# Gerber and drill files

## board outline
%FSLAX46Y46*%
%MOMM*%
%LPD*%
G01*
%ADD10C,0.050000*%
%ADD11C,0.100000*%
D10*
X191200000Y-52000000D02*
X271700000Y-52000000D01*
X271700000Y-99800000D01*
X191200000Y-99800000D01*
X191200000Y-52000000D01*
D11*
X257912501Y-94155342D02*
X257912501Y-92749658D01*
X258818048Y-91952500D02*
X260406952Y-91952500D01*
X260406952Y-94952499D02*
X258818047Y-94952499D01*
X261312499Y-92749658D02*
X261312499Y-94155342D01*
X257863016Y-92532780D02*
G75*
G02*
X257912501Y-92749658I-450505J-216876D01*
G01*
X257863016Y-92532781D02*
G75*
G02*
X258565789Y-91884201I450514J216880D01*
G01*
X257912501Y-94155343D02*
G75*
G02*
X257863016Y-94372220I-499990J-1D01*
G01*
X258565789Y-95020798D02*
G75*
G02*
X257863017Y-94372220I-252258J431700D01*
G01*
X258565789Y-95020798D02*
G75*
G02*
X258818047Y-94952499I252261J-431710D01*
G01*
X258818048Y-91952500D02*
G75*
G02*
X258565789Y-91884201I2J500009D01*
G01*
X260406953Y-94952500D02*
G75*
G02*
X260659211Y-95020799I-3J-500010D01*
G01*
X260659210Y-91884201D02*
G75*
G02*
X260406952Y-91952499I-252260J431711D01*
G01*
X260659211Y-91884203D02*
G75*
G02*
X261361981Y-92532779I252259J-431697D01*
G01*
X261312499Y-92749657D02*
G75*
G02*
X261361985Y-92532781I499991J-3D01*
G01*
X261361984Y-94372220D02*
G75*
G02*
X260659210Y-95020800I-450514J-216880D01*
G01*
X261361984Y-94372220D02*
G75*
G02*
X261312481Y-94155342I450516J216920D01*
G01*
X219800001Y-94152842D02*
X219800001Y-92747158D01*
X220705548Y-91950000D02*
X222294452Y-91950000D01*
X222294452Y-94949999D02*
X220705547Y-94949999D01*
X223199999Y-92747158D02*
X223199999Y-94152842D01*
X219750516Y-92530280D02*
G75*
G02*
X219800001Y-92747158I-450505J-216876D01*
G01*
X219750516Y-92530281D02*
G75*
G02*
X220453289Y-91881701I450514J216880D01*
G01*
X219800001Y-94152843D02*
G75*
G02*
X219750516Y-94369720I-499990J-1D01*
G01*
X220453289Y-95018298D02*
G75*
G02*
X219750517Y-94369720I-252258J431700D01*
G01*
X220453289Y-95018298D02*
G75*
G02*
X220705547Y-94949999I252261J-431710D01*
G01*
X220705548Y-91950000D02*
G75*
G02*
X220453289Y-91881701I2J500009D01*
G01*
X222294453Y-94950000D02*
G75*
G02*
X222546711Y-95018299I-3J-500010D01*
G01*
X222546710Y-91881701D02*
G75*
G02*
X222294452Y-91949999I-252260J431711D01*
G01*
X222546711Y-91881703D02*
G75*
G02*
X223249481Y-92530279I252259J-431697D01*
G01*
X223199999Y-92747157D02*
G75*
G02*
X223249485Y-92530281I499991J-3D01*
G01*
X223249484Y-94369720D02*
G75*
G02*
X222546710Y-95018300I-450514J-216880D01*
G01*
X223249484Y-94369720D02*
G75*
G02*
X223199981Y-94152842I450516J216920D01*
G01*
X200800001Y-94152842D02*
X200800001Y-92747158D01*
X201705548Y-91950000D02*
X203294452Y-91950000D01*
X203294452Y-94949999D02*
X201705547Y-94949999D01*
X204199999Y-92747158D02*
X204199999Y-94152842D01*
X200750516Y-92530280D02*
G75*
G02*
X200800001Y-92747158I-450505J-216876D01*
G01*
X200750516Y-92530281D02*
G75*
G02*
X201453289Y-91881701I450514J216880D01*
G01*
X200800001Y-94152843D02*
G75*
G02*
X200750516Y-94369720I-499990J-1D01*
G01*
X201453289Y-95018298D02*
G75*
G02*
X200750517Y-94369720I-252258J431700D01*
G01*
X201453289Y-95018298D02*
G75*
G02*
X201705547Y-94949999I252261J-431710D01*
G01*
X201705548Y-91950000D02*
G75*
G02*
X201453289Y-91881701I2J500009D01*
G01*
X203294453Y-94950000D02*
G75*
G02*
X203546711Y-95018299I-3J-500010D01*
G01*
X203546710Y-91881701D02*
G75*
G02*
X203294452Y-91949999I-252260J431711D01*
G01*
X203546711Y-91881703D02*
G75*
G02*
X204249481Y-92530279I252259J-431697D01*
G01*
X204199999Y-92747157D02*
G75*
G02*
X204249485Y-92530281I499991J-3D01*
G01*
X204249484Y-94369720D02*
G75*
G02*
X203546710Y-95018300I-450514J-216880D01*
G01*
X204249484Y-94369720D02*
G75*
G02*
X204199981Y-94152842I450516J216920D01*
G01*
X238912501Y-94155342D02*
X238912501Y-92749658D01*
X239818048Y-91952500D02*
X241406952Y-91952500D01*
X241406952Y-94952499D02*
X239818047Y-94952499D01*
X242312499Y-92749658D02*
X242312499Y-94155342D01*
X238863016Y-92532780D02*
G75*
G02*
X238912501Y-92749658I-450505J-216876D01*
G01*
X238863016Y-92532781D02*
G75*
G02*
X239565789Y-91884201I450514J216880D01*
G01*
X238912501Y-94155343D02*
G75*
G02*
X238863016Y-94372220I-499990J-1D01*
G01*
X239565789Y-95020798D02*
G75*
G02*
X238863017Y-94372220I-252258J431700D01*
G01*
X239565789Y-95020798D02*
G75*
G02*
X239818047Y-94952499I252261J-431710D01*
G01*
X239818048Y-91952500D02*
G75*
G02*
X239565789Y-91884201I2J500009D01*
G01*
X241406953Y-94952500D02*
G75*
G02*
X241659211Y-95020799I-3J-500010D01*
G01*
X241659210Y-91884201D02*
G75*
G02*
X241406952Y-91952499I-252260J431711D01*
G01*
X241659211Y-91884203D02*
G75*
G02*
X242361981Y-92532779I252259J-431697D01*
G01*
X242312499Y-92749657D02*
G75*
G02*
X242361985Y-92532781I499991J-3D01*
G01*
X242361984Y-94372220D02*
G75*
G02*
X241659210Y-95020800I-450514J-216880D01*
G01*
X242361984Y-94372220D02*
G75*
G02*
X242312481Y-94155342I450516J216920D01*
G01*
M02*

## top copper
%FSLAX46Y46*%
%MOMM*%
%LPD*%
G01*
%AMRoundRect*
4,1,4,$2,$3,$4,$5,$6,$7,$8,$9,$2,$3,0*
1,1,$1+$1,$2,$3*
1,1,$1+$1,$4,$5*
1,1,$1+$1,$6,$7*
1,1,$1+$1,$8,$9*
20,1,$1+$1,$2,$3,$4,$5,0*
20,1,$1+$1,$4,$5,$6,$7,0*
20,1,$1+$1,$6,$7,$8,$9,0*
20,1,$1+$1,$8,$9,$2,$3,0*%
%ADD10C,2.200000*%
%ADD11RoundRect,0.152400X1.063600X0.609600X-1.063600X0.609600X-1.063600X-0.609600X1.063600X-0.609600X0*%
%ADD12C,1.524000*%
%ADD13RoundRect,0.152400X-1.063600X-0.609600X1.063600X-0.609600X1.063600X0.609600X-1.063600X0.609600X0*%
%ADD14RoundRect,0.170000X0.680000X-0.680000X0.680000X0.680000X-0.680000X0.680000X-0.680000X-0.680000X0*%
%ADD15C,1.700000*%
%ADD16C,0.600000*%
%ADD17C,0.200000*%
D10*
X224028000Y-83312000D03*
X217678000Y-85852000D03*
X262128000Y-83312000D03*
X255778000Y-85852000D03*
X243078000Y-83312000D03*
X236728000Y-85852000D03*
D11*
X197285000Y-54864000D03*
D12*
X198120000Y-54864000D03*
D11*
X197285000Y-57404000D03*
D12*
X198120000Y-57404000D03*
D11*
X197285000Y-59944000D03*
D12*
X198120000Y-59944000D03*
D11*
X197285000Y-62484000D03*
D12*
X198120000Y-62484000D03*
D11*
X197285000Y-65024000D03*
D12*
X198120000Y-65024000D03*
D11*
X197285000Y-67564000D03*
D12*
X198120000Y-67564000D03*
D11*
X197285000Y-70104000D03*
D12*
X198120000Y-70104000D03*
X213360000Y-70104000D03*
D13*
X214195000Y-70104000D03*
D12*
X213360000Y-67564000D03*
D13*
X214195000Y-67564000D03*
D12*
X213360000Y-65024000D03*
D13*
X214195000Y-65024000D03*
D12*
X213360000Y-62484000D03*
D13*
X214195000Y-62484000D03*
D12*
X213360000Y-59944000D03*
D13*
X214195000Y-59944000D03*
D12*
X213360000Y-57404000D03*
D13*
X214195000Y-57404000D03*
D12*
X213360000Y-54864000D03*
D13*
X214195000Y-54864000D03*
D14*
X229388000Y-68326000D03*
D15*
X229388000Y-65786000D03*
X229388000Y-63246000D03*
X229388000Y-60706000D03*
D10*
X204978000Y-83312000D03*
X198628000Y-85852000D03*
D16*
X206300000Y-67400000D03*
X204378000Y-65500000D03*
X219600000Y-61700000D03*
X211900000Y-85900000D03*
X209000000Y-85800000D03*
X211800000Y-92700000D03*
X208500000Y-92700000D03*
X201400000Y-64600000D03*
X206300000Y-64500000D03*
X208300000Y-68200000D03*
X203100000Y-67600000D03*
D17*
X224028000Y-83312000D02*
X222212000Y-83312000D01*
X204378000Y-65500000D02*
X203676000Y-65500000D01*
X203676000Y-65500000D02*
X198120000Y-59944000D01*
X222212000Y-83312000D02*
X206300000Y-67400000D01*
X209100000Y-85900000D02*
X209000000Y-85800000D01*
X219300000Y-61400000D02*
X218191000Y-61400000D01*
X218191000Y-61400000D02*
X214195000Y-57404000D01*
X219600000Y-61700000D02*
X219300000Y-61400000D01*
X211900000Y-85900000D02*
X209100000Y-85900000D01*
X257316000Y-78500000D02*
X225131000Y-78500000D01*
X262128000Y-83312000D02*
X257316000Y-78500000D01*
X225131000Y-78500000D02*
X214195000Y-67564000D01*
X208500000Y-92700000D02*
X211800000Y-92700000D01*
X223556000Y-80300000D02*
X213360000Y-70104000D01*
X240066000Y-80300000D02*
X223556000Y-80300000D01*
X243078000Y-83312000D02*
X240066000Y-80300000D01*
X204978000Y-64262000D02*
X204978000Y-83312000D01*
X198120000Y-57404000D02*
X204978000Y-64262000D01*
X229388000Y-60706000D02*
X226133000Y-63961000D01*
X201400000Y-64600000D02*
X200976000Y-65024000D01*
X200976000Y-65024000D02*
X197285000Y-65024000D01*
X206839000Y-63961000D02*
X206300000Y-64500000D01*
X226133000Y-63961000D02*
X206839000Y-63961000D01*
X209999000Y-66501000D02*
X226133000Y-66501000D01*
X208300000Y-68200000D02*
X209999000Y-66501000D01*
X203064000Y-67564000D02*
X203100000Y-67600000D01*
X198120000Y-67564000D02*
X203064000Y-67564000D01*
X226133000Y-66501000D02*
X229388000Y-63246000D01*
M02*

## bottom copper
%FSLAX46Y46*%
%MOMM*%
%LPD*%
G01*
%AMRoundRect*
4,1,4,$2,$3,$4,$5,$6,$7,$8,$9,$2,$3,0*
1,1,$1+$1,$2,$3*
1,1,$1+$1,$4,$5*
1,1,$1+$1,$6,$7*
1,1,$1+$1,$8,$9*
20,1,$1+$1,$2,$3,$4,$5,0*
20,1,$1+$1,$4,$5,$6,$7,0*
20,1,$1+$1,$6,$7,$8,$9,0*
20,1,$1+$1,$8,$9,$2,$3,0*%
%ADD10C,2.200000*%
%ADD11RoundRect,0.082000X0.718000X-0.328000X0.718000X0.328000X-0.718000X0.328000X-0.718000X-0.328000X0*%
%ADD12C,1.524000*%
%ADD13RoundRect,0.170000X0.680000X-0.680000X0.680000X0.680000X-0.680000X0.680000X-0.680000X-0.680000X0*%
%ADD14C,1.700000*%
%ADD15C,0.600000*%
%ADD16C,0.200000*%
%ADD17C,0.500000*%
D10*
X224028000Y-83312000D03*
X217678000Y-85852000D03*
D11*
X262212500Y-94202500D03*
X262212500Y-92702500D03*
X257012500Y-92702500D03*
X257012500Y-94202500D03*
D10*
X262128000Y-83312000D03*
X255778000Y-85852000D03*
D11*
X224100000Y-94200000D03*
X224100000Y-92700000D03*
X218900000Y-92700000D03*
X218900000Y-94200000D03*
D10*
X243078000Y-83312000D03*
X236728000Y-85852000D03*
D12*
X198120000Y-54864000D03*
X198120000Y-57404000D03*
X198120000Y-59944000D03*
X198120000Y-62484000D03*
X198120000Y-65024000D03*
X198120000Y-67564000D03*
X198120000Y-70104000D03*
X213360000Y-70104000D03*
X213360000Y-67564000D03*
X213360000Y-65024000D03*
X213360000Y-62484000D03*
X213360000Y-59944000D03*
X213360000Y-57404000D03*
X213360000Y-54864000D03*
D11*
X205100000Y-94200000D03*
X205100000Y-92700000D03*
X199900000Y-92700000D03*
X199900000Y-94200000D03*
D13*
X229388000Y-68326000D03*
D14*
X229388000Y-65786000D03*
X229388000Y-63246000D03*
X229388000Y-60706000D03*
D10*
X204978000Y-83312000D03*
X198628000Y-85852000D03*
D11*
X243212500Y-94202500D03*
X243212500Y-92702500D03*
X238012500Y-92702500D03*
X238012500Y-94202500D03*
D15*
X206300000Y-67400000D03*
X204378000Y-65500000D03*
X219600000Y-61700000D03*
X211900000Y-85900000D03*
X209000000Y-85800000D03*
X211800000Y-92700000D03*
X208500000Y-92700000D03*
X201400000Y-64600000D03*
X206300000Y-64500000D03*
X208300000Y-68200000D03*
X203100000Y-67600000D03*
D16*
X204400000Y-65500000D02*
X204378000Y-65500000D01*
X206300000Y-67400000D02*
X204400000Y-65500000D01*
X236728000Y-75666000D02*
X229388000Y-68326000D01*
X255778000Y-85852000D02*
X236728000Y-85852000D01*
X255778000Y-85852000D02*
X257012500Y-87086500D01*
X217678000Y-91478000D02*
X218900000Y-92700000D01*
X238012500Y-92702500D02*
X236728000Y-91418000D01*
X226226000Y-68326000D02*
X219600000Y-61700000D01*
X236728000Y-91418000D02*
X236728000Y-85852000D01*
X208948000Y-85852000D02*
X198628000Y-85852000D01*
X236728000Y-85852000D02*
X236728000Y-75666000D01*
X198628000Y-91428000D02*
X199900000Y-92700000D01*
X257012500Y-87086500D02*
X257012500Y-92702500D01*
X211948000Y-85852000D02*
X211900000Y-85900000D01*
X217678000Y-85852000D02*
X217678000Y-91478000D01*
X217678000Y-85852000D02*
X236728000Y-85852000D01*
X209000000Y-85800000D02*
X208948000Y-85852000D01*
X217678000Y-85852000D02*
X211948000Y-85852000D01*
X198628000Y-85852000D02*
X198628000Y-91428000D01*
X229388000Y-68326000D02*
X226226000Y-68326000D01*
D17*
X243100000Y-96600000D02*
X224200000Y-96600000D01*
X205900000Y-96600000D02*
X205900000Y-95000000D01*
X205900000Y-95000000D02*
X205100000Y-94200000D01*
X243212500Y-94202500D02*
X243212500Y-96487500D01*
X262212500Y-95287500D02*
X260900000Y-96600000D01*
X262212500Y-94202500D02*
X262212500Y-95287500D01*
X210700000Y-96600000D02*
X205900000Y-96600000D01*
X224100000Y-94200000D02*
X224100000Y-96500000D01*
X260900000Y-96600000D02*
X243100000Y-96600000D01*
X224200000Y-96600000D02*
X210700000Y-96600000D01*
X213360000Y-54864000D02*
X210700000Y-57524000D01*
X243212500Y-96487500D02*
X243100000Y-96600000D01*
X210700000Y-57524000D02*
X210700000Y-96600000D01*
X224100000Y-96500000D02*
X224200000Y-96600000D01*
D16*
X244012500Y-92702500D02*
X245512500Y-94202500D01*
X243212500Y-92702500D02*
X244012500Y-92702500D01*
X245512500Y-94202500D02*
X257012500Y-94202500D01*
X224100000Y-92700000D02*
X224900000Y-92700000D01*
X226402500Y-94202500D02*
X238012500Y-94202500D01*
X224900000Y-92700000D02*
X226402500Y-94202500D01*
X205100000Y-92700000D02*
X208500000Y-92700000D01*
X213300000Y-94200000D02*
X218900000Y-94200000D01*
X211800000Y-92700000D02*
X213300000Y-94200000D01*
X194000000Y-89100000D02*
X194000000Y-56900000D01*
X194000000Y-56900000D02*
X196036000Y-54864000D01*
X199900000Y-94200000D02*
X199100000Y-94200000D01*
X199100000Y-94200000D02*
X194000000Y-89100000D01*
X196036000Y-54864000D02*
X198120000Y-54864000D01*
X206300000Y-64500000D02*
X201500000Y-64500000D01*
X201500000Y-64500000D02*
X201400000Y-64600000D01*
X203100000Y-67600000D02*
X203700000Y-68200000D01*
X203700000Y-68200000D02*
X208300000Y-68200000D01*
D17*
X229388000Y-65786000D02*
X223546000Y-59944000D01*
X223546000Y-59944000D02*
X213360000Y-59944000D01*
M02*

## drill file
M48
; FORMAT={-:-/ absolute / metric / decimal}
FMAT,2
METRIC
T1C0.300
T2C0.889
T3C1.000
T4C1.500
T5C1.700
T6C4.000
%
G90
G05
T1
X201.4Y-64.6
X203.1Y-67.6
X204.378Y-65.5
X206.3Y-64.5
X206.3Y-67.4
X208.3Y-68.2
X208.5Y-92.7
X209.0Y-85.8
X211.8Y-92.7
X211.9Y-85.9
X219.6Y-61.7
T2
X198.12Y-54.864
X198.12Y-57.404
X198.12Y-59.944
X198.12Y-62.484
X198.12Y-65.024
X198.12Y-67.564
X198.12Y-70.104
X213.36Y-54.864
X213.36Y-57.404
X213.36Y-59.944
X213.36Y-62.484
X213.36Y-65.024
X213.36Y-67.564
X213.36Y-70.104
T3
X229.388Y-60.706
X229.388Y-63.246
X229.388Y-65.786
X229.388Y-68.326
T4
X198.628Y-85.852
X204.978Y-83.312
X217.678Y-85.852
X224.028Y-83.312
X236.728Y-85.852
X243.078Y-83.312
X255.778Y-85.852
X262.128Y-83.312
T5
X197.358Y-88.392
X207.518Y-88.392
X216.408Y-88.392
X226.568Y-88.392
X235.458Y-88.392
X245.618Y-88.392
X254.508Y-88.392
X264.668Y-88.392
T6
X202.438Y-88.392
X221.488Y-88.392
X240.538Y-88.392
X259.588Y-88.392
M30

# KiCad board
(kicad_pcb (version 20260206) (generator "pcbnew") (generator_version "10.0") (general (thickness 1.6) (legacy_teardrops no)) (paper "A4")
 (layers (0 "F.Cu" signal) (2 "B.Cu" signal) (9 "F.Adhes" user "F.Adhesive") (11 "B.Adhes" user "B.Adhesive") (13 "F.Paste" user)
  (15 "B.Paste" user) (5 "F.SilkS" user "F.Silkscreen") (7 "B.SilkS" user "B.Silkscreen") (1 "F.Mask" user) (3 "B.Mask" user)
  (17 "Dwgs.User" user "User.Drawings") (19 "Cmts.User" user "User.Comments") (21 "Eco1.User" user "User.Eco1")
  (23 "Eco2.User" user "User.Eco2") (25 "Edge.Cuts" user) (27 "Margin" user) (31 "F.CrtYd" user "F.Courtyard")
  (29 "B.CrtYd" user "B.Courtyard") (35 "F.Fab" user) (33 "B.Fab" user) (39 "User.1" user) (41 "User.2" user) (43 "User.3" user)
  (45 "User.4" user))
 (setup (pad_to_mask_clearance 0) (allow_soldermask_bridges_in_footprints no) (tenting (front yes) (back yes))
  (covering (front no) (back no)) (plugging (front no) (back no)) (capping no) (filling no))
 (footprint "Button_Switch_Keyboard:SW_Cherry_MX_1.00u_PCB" (layer "F.Cu") (at 224.028 83.312)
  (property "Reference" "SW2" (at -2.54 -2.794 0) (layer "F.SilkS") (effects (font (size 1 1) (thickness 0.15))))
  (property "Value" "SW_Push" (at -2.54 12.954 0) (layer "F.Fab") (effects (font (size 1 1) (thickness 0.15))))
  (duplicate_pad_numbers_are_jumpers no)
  (pad "" np_thru_hole circle (at -7.62 5.08) (size 1.7 1.7) (drill 1.7) (layers "*.Cu" "*.Mask"))
  (pad "" np_thru_hole circle (at -2.54 5.08) (size 4 4) (drill 4) (layers "*.Cu" "*.Mask"))
  (pad "" np_thru_hole circle (at 2.54 5.08) (size 1.7 1.7) (drill 1.7) (layers "*.Cu" "*.Mask"))
  (pad "1" thru_hole circle (at 0 0) (size 2.2 2.2) (drill 1.5) (layers "*.Cu" "*.Mask") (remove_unused_layers no)
   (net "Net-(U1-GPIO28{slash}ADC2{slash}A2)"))
  (pad "2" thru_hole circle (at -6.35 2.54) (size 2.2 2.2) (drill 1.5) (layers "*.Cu" "*.Mask") (remove_unused_layers no) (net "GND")))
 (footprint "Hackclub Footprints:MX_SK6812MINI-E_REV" (layer "F.Cu") (at 259.6125 88.3725)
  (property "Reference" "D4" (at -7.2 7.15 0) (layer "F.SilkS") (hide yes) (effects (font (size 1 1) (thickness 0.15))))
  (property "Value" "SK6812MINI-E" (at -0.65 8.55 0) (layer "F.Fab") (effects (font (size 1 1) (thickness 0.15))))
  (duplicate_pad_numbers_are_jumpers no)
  (fp_line (start -1.699999 5.782842) (end -1.699999 4.377158) (stroke (width 0.1) (type solid)) (layer "Edge.Cuts"))
  (fp_line (start -0.794452 3.58) (end 0.794452 3.58) (stroke (width 0.1) (type solid)) (layer "Edge.Cuts"))
  (fp_line (start 0.794452 6.579999) (end -0.794453 6.579999) (stroke (width 0.1) (type solid)) (layer "Edge.Cuts"))
  (fp_line (start 1.699999 4.377158) (end 1.699999 5.782842) (stroke (width 0.1) (type solid)) (layer "Edge.Cuts"))
  (fp_arc (start -1.749484 4.16028) (mid -1.712527 4.265932) (end -1.699999 4.377158) (stroke (width 0.1) (type solid)) (layer "Edge.Cuts"))
  (fp_arc (start -1.749484 4.160281) (mid -1.638072 3.575965) (end -1.046711 3.511701) (stroke (width 0.1) (type solid)) (layer "Edge.Cuts"))
  (fp_arc (start -1.699999 5.782843) (mid -1.712527 5.894068) (end -1.749484 5.99972) (stroke (width 0.1) (type solid)) (layer "Edge.Cuts"))
  (fp_arc (start -1.046711 6.648298) (mid -1.638071 6.584034) (end -1.749484 5.99972) (stroke (width 0.1) (type solid)) (layer "Edge.Cuts"))
  (fp_arc (start -1.046711 6.648298) (mid -0.925123 6.597376) (end -0.794453 6.579999) (stroke (width 0.1) (type solid)) (layer "Edge.Cuts"))
  (fp_arc (start -0.794452 3.58) (mid -0.925123 3.562623) (end -1.046711 3.511701) (stroke (width 0.1) (type solid)) (layer "Edge.Cuts"))
  (fp_arc (start 0.794453 6.58) (mid 0.925123 6.597377) (end 1.046711 6.648299) (stroke (width 0.1) (type solid)) (layer "Edge.Cuts"))
  (fp_arc (start 1.04671 3.511701) (mid 0.925122 3.562623) (end 0.794452 3.58) (stroke (width 0.1) (type solid)) (layer "Edge.Cuts"))
  (fp_arc (start 1.046711 3.511703) (mid 1.63807 3.575966) (end 1.749484 4.16028) (stroke (width 0.1) (type solid)) (layer "Edge.Cuts"))
  (fp_arc (start 1.699999 4.377157) (mid 1.712527 4.265932) (end 1.749484 4.16028) (stroke (width 0.1) (type solid)) (layer "Edge.Cuts"))
  (fp_arc (start 1.749484 5.99972) (mid 1.638071 6.584035) (end 1.046711 6.648299) (stroke (width 0.1) (type solid)) (layer "Edge.Cuts"))
  (fp_arc (start 1.749484 5.99972) (mid 1.712527 5.894068) (end 1.699999 5.782842) (stroke (width 0.1) (type solid)) (layer "Edge.Cuts"))
  (pad "1" smd roundrect (at 2.6 5.83 90) (size 0.82 1.6) (layers "B.Cu" "B.Mask" "B.Paste") (roundrect_rratio 0.1) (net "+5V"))
  (pad "2" smd roundrect (at 2.6 4.33 90) (size 0.82 1.6) (layers "B.Cu" "B.Mask" "B.Paste") (roundrect_rratio 0.1)
   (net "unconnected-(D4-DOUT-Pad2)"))
  (pad "3" smd roundrect (at -2.6 4.33 90) (size 0.82 1.6) (layers "B.Cu" "B.Mask" "B.Paste") (roundrect_rratio 0.1) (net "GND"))
  (pad "4" smd roundrect (at -2.6 5.83 90) (size 0.82 1.6) (layers "B.Cu" "B.Mask" "B.Paste") (roundrect_rratio 0.1) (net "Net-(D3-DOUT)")))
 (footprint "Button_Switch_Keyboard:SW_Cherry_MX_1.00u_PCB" (layer "F.Cu") (at 262.128 83.312)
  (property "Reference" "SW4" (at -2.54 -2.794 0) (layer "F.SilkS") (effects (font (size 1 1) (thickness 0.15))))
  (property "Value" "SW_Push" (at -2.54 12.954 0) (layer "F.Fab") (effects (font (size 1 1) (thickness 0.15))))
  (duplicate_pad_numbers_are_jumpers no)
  (pad "" np_thru_hole circle (at -7.62 5.08) (size 1.7 1.7) (drill 1.7) (layers "*.Cu" "*.Mask"))
  (pad "" np_thru_hole circle (at -2.54 5.08) (size 4 4) (drill 4) (layers "*.Cu" "*.Mask"))
  (pad "" np_thru_hole circle (at 2.54 5.08) (size 1.7 1.7) (drill 1.7) (layers "*.Cu" "*.Mask"))
  (pad "1" thru_hole circle (at 0 0) (size 2.2 2.2) (drill 1.5) (layers "*.Cu" "*.Mask") (remove_unused_layers no)
   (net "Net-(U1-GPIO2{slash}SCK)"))
  (pad "2" thru_hole circle (at -6.35 2.54) (size 2.2 2.2) (drill 1.5) (layers "*.Cu" "*.Mask") (remove_unused_layers no) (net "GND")))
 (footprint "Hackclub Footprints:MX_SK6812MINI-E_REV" (layer "F.Cu") (at 221.5 88.37)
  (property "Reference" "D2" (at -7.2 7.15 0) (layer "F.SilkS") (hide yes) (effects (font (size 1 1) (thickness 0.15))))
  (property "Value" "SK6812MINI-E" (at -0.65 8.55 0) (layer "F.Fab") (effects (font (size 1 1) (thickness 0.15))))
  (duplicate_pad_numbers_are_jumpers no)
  (fp_line (start -1.699999 5.782842) (end -1.699999 4.377158) (stroke (width 0.1) (type solid)) (layer "Edge.Cuts"))
  (fp_line (start -0.794452 3.58) (end 0.794452 3.58) (stroke (width 0.1) (type solid)) (layer "Edge.Cuts"))
  (fp_line (start 0.794452 6.579999) (end -0.794453 6.579999) (stroke (width 0.1) (type solid)) (layer "Edge.Cuts"))
  (fp_line (start 1.699999 4.377158) (end 1.699999 5.782842) (stroke (width 0.1) (type solid)) (layer "Edge.Cuts"))
  (fp_arc (start -1.749484 4.16028) (mid -1.712527 4.265932) (end -1.699999 4.377158) (stroke (width 0.1) (type solid)) (layer "Edge.Cuts"))
  (fp_arc (start -1.749484 4.160281) (mid -1.638072 3.575965) (end -1.046711 3.511701) (stroke (width 0.1) (type solid)) (layer "Edge.Cuts"))
  (fp_arc (start -1.699999 5.782843) (mid -1.712527 5.894068) (end -1.749484 5.99972) (stroke (width 0.1) (type solid)) (layer "Edge.Cuts"))
  (fp_arc (start -1.046711 6.648298) (mid -1.638071 6.584034) (end -1.749484 5.99972) (stroke (width 0.1) (type solid)) (layer "Edge.Cuts"))
  (fp_arc (start -1.046711 6.648298) (mid -0.925123 6.597376) (end -0.794453 6.579999) (stroke (width 0.1) (type solid)) (layer "Edge.Cuts"))
  (fp_arc (start -0.794452 3.58) (mid -0.925123 3.562623) (end -1.046711 3.511701) (stroke (width 0.1) (type solid)) (layer "Edge.Cuts"))
  (fp_arc (start 0.794453 6.58) (mid 0.925123 6.597377) (end 1.046711 6.648299) (stroke (width 0.1) (type solid)) (layer "Edge.Cuts"))
  (fp_arc (start 1.04671 3.511701) (mid 0.925122 3.562623) (end 0.794452 3.58) (stroke (width 0.1) (type solid)) (layer "Edge.Cuts"))
  (fp_arc (start 1.046711 3.511703) (mid 1.63807 3.575966) (end 1.749484 4.16028) (stroke (width 0.1) (type solid)) (layer "Edge.Cuts"))
  (fp_arc (start 1.699999 4.377157) (mid 1.712527 4.265932) (end 1.749484 4.16028) (stroke (width 0.1) (type solid)) (layer "Edge.Cuts"))
  (fp_arc (start 1.749484 5.99972) (mid 1.638071 6.584035) (end 1.046711 6.648299) (stroke (width 0.1) (type solid)) (layer "Edge.Cuts"))
  (fp_arc (start 1.749484 5.99972) (mid 1.712527 5.894068) (end 1.699999 5.782842) (stroke (width 0.1) (type solid)) (layer "Edge.Cuts"))
  (pad "1" smd roundrect (at 2.6 5.83 90) (size 0.82 1.6) (layers "B.Cu" "B.Mask" "B.Paste") (roundrect_rratio 0.1) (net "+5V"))
  (pad "2" smd roundrect (at 2.6 4.33 90) (size 0.82 1.6) (layers "B.Cu" "B.Mask" "B.Paste") (roundrect_rratio 0.1) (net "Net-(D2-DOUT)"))
  (pad "3" smd roundrect (at -2.6 4.33 90) (size 0.82 1.6) (layers "B.Cu" "B.Mask" "B.Paste") (roundrect_rratio 0.1) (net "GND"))
  (pad "4" smd roundrect (at -2.6 5.83 90) (size 0.82 1.6) (layers "B.Cu" "B.Mask" "B.Paste") (roundrect_rratio 0.1) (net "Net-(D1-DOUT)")))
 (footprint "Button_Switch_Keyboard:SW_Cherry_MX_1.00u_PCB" (layer "F.Cu") (at 243.078 83.312)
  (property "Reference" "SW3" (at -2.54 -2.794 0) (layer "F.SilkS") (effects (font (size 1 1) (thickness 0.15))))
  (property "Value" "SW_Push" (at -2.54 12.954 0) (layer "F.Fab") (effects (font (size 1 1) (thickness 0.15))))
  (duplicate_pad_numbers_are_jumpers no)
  (pad "" np_thru_hole circle (at -7.62 5.08) (size 1.7 1.7) (drill 1.7) (layers "*.Cu" "*.Mask"))
  (pad "" np_thru_hole circle (at -2.54 5.08) (size 4 4) (drill 4) (layers "*.Cu" "*.Mask"))
  (pad "" np_thru_hole circle (at 2.54 5.08) (size 1.7 1.7) (drill 1.7) (layers "*.Cu" "*.Mask"))
  (pad "1" thru_hole circle (at 0 0) (size 2.2 2.2) (drill 1.5) (layers "*.Cu" "*.Mask") (remove_unused_layers no)
   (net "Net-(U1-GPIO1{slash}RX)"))
  (pad "2" thru_hole circle (at -6.35 2.54) (size 2.2 2.2) (drill 1.5) (layers "*.Cu" "*.Mask") (remove_unused_layers no) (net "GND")))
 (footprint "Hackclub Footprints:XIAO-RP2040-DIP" (layer "F.Cu") (at 205.74 62.484)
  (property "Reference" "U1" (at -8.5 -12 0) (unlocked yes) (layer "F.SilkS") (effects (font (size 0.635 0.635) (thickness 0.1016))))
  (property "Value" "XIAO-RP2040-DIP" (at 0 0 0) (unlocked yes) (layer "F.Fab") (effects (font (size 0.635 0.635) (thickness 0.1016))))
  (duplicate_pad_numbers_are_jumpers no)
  (pad "1" smd roundrect (at -8.455 -7.62 180) (size 2.432 1.524) (layers "F.Cu" "F.Mask") (roundrect_rratio 0.1) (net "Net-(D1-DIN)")
   (thermal_bridge_angle 45))
  (pad "1" thru_hole circle (at -7.62 -7.62 180) (size 1.524 1.524) (drill 0.889) (layers "*.Cu" "*.Mask") (remove_unused_layers no)
   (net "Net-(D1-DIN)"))
  (pad "2" smd roundrect (at -8.455 -5.08 180) (size 2.432 1.524) (layers "F.Cu" "F.Mask") (roundrect_rratio 0.1)
   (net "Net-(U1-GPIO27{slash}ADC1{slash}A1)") (thermal_bridge_angle 45))
  (pad "2" thru_hole circle (at -7.62 -5.08 180) (size 1.524 1.524) (drill 0.889) (layers "*.Cu" "*.Mask") (remove_unused_layers no)
   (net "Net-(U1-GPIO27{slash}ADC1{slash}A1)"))
  (pad "3" smd roundrect (at -8.455 -2.54 180) (size 2.432 1.524) (layers "F.Cu" "F.Mask") (roundrect_rratio 0.1)
   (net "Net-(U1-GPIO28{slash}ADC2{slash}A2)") (thermal_bridge_angle 45))
  (pad "3" thru_hole circle (at -7.62 -2.54 180) (size 1.524 1.524) (drill 0.889) (layers "*.Cu" "*.Mask") (remove_unused_layers no)
   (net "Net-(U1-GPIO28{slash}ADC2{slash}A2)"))
  (pad "4" smd roundrect (at -8.455 0 180) (size 2.432 1.524) (layers "F.Cu" "F.Mask") (roundrect_rratio 0.1)
   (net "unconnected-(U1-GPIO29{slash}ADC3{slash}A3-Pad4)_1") (thermal_bridge_angle 45))
  (pad "4" thru_hole circle (at -7.62 0 180) (size 1.524 1.524) (drill 0.889) (layers "*.Cu" "*.Mask") (remove_unused_layers no)
   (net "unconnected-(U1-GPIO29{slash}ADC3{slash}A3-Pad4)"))
  (pad "5" smd roundrect (at -8.455 2.54 180) (size 2.432 1.524) (layers "F.Cu" "F.Mask") (roundrect_rratio 0.1) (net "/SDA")
   (thermal_bridge_angle 45))
  (pad "5" thru_hole circle (at -7.62 2.54 180) (size 1.524 1.524) (drill 0.889) (layers "*.Cu" "*.Mask") (remove_unused_layers no)
   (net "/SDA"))
  (pad "6" smd roundrect (at -8.455 5.08 180) (size 2.432 1.524) (layers "F.Cu" "F.Mask") (roundrect_rratio 0.1) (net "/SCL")
   (thermal_bridge_angle 45))
  (pad "6" thru_hole circle (at -7.62 5.08 180) (size 1.524 1.524) (drill 0.889) (layers "*.Cu" "*.Mask") (remove_unused_layers no)
   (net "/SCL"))
  (pad "7" smd roundrect (at -8.455 7.62 180) (size 2.432 1.524) (layers "F.Cu" "F.Mask") (roundrect_rratio 0.1)
   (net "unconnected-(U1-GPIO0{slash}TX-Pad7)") (thermal_bridge_angle 45))
  (pad "7" thru_hole circle (at -7.62 7.62 180) (size 1.524 1.524) (drill 0.889) (layers "*.Cu" "*.Mask") (remove_unused_layers no)
   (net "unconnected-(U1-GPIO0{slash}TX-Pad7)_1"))
  (pad "8" thru_hole circle (at 7.62 7.62) (size 1.524 1.524) (drill 0.889) (layers "*.Cu" "*.Mask") (remove_unused_layers no)
   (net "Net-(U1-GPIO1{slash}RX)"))
  (pad "8" smd roundrect (at 8.455 7.62) (size 2.432 1.524) (layers "F.Cu" "F.Mask") (roundrect_rratio 0.1) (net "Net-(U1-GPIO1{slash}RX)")
   (thermal_bridge_angle 45))
  (pad "9" thru_hole circle (at 7.62 5.08) (size 1.524 1.524) (drill 0.889) (layers "*.Cu" "*.Mask") (remove_unused_layers no)
   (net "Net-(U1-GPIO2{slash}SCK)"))
  (pad "9" smd roundrect (at 8.455 5.08) (size 2.432 1.524) (layers "F.Cu" "F.Mask") (roundrect_rratio 0.1) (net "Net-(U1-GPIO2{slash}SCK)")
   (thermal_bridge_angle 45))
  (pad "10" thru_hole circle (at 7.62 2.54) (size 1.524 1.524) (drill 0.889) (layers "*.Cu" "*.Mask") (remove_unused_layers no)
   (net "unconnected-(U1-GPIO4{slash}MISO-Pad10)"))
  (pad "10" smd roundrect (at 8.455 2.54) (size 2.432 1.524) (layers "F.Cu" "F.Mask") (roundrect_rratio 0.1)
   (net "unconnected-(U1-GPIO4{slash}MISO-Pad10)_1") (thermal_bridge_angle 45))
  (pad "11" thru_hole circle (at 7.62 0) (size 1.524 1.524) (drill 0.889) (layers "*.Cu" "*.Mask") (remove_unused_layers no)
   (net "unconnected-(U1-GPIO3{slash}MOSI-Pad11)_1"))
  (pad "11" smd roundrect (at 8.455 0) (size 2.432 1.524) (layers "F.Cu" "F.Mask") (roundrect_rratio 0.1)
   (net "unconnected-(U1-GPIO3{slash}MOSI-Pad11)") (thermal_bridge_angle 45))
  (pad "12" thru_hole circle (at 7.62 -2.54) (size 1.524 1.524) (drill 0.889) (layers "*.Cu" "*.Mask") (remove_unused_layers no)
   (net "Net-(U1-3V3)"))
  (pad "12" smd roundrect (at 8.455 -2.54) (size 2.432 1.524) (layers "F.Cu" "F.Mask") (roundrect_rratio 0.1) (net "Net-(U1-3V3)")
   (thermal_bridge_angle 45))
  (pad "13" thru_hole circle (at 7.62 -5.08) (size 1.524 1.524) (drill 0.889) (layers "*.Cu" "*.Mask") (remove_unused_layers no) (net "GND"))
  (pad "13" smd roundrect (at 8.455 -5.08) (size 2.432 1.524) (layers "F.Cu" "F.Mask") (roundrect_rratio 0.1) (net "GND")
   (thermal_bridge_angle 45))
  (pad "14" thru_hole circle (at 7.62 -7.62) (size 1.524 1.524) (drill 0.889) (layers "*.Cu" "*.Mask") (remove_unused_layers no) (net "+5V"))
  (pad "14" smd roundrect (at 8.455 -7.62) (size 2.432 1.524) (layers "F.Cu" "F.Mask") (roundrect_rratio 0.1) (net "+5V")
   (thermal_bridge_angle 45)))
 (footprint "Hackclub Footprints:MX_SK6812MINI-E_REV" (layer "F.Cu") (at 202.5 88.37)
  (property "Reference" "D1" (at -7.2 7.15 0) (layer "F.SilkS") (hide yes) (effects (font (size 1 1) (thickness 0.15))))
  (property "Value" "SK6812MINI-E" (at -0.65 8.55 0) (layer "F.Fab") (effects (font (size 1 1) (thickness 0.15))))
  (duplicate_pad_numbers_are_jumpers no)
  (fp_line (start -1.699999 5.782842) (end -1.699999 4.377158) (stroke (width 0.1) (type solid)) (layer "Edge.Cuts"))
  (fp_line (start -0.794452 3.58) (end 0.794452 3.58) (stroke (width 0.1) (type solid)) (layer "Edge.Cuts"))
  (fp_line (start 0.794452 6.579999) (end -0.794453 6.579999) (stroke (width 0.1) (type solid)) (layer "Edge.Cuts"))
  (fp_line (start 1.699999 4.377158) (end 1.699999 5.782842) (stroke (width 0.1) (type solid)) (layer "Edge.Cuts"))
  (fp_arc (start -1.749484 4.16028) (mid -1.712527 4.265932) (end -1.699999 4.377158) (stroke (width 0.1) (type solid)) (layer "Edge.Cuts"))
  (fp_arc (start -1.749484 4.160281) (mid -1.638072 3.575965) (end -1.046711 3.511701) (stroke (width 0.1) (type solid)) (layer "Edge.Cuts"))
  (fp_arc (start -1.699999 5.782843) (mid -1.712527 5.894068) (end -1.749484 5.99972) (stroke (width 0.1) (type solid)) (layer "Edge.Cuts"))
  (fp_arc (start -1.046711 6.648298) (mid -1.638071 6.584034) (end -1.749484 5.99972) (stroke (width 0.1) (type solid)) (layer "Edge.Cuts"))
  (fp_arc (start -1.046711 6.648298) (mid -0.925123 6.597376) (end -0.794453 6.579999) (stroke (width 0.1) (type solid)) (layer "Edge.Cuts"))
  (fp_arc (start -0.794452 3.58) (mid -0.925123 3.562623) (end -1.046711 3.511701) (stroke (width 0.1) (type solid)) (layer "Edge.Cuts"))
  (fp_arc (start 0.794453 6.58) (mid 0.925123 6.597377) (end 1.046711 6.648299) (stroke (width 0.1) (type solid)) (layer "Edge.Cuts"))
  (fp_arc (start 1.04671 3.511701) (mid 0.925122 3.562623) (end 0.794452 3.58) (stroke (width 0.1) (type solid)) (layer "Edge.Cuts"))
  (fp_arc (start 1.046711 3.511703) (mid 1.63807 3.575966) (end 1.749484 4.16028) (stroke (width 0.1) (type solid)) (layer "Edge.Cuts"))
  (fp_arc (start 1.699999 4.377157) (mid 1.712527 4.265932) (end 1.749484 4.16028) (stroke (width 0.1) (type solid)) (layer "Edge.Cuts"))
  (fp_arc (start 1.749484 5.99972) (mid 1.638071 6.584035) (end 1.046711 6.648299) (stroke (width 0.1) (type solid)) (layer "Edge.Cuts"))
  (fp_arc (start 1.749484 5.99972) (mid 1.712527 5.894068) (end 1.699999 5.782842) (stroke (width 0.1) (type solid)) (layer "Edge.Cuts"))
  (pad "1" smd roundrect (at 2.6 5.83 90) (size 0.82 1.6) (layers "B.Cu" "B.Mask" "B.Paste") (roundrect_rratio 0.1) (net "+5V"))
  (pad "2" smd roundrect (at 2.6 4.33 90) (size 0.82 1.6) (layers "B.Cu" "B.Mask" "B.Paste") (roundrect_rratio 0.1) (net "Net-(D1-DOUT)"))
  (pad "3" smd roundrect (at -2.6 4.33 90) (size 0.82 1.6) (layers "B.Cu" "B.Mask" "B.Paste") (roundrect_rratio 0.1) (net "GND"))
  (pad "4" smd roundrect (at -2.6 5.83 90) (size 0.82 1.6) (layers "B.Cu" "B.Mask" "B.Paste") (roundrect_rratio 0.1) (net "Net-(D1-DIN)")))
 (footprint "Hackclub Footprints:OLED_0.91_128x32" (layer "F.Cu") (at 229.388 68.326 90)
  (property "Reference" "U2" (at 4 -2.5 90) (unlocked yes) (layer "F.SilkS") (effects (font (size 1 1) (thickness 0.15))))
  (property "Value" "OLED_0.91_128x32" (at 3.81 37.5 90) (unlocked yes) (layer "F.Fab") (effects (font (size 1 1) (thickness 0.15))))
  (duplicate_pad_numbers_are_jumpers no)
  (pad "1" thru_hole roundrect (at 0 0 90) (size 1.7 1.7) (drill 1) (layers "*.Cu" "*.Mask") (remove_unused_layers no)
   (roundrect_rratio 0.1) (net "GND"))
  (pad "2" thru_hole circle (at 2.54 0 90) (size 1.7 1.7) (drill 1) (layers "*.Cu" "*.Mask") (remove_unused_layers no) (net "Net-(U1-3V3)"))
  (pad "3" thru_hole circle (at 5.08 0 90) (size 1.7 1.7) (drill 1) (layers "*.Cu" "*.Mask") (remove_unused_layers no) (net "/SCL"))
  (pad "4" thru_hole circle (at 7.62 0 90) (size 1.7 1.7) (drill 1) (layers "*.Cu" "*.Mask") (remove_unused_layers no) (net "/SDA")))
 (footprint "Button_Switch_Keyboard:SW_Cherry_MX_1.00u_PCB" (layer "F.Cu") (at 204.978 83.312)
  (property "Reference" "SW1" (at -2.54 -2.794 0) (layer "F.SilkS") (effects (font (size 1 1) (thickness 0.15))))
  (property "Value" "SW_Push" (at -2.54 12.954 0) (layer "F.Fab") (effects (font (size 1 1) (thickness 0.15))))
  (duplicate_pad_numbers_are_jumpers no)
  (pad "" np_thru_hole circle (at -7.62 5.08) (size 1.7 1.7) (drill 1.7) (layers "*.Cu" "*.Mask"))
  (pad "" np_thru_hole circle (at -2.54 5.08) (size 4 4) (drill 4) (layers "*.Cu" "*.Mask"))
  (pad "" np_thru_hole circle (at 2.54 5.08) (size 1.7 1.7) (drill 1.7) (layers "*.Cu" "*.Mask"))
  (pad "1" thru_hole circle (at 0 0) (size 2.2 2.2) (drill 1.5) (layers "*.Cu" "*.Mask") (remove_unused_layers no)
   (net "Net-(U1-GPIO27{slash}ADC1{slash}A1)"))
  (pad "2" thru_hole circle (at -6.35 2.54) (size 2.2 2.2) (drill 1.5) (layers "*.Cu" "*.Mask") (remove_unused_layers no) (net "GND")))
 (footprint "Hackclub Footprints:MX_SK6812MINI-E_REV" (layer "F.Cu") (at 240.6125 88.3725)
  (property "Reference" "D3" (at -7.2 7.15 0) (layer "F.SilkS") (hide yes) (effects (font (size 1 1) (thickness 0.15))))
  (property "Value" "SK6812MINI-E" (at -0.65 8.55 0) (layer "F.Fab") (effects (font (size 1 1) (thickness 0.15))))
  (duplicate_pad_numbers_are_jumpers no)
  (fp_line (start -1.699999 5.782842) (end -1.699999 4.377158) (stroke (width 0.1) (type solid)) (layer "Edge.Cuts"))
  (fp_line (start -0.794452 3.58) (end 0.794452 3.58) (stroke (width 0.1) (type solid)) (layer "Edge.Cuts"))
  (fp_line (start 0.794452 6.579999) (end -0.794453 6.579999) (stroke (width 0.1) (type solid)) (layer "Edge.Cuts"))
  (fp_line (start 1.699999 4.377158) (end 1.699999 5.782842) (stroke (width 0.1) (type solid)) (layer "Edge.Cuts"))
  (fp_arc (start -1.749484 4.16028) (mid -1.712527 4.265932) (end -1.699999 4.377158) (stroke (width 0.1) (type solid)) (layer "Edge.Cuts"))
  (fp_arc (start -1.749484 4.160281) (mid -1.638072 3.575965) (end -1.046711 3.511701) (stroke (width 0.1) (type solid)) (layer "Edge.Cuts"))
  (fp_arc (start -1.699999 5.782843) (mid -1.712527 5.894068) (end -1.749484 5.99972) (stroke (width 0.1) (type solid)) (layer "Edge.Cuts"))
  (fp_arc (start -1.046711 6.648298) (mid -1.638071 6.584034) (end -1.749484 5.99972) (stroke (width 0.1) (type solid)) (layer "Edge.Cuts"))
  (fp_arc (start -1.046711 6.648298) (mid -0.925123 6.597376) (end -0.794453 6.579999) (stroke (width 0.1) (type solid)) (layer "Edge.Cuts"))
  (fp_arc (start -0.794452 3.58) (mid -0.925123 3.562623) (end -1.046711 3.511701) (stroke (width 0.1) (type solid)) (layer "Edge.Cuts"))
  (fp_arc (start 0.794453 6.58) (mid 0.925123 6.597377) (end 1.046711 6.648299) (stroke (width 0.1) (type solid)) (layer "Edge.Cuts"))
  (fp_arc (start 1.04671 3.511701) (mid 0.925122 3.562623) (end 0.794452 3.58) (stroke (width 0.1) (type solid)) (layer "Edge.Cuts"))
  (fp_arc (start 1.046711 3.511703) (mid 1.63807 3.575966) (end 1.749484 4.16028) (stroke (width 0.1) (type solid)) (layer "Edge.Cuts"))
  (fp_arc (start 1.699999 4.377157) (mid 1.712527 4.265932) (end 1.749484 4.16028) (stroke (width 0.1) (type solid)) (layer "Edge.Cuts"))
  (fp_arc (start 1.749484 5.99972) (mid 1.638071 6.584035) (end 1.046711 6.648299) (stroke (width 0.1) (type solid)) (layer "Edge.Cuts"))
  (fp_arc (start 1.749484 5.99972) (mid 1.712527 5.894068) (end 1.699999 5.782842) (stroke (width 0.1) (type solid)) (layer "Edge.Cuts"))
  (pad "1" smd roundrect (at 2.6 5.83 90) (size 0.82 1.6) (layers "B.Cu" "B.Mask" "B.Paste") (roundrect_rratio 0.1) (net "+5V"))
  (pad "2" smd roundrect (at 2.6 4.33 90) (size 0.82 1.6) (layers "B.Cu" "B.Mask" "B.Paste") (roundrect_rratio 0.1) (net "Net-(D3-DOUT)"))
  (pad "3" smd roundrect (at -2.6 4.33 90) (size 0.82 1.6) (layers "B.Cu" "B.Mask" "B.Paste") (roundrect_rratio 0.1) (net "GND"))
  (pad "4" smd roundrect (at -2.6 5.83 90) (size 0.82 1.6) (layers "B.Cu" "B.Mask" "B.Paste") (roundrect_rratio 0.1) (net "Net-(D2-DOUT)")))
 (gr_rect (start 191.2 52) (end 271.7 99.8) (stroke (width 0.05) (type default)) (fill no) (layer "Edge.Cuts"))
 (segment (start 224.028 83.312) (end 222.212 83.312) (width 0.2) (layer "F.Cu") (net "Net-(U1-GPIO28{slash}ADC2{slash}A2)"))
 (segment (start 204.378 65.5) (end 203.676 65.5) (width 0.2) (layer "F.Cu") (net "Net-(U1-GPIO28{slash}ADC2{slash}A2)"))
 (segment (start 203.676 65.5) (end 198.12 59.944) (width 0.2) (layer "F.Cu") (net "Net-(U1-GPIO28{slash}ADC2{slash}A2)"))
 (segment (start 222.212 83.312) (end 206.3 67.4) (width 0.2) (layer "F.Cu") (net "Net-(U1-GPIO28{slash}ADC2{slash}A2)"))
 (via (at 206.3 67.4) (size 0.6) (drill 0.3) (layers "F.Cu" "B.Cu") (capping no) (covering (front no) (back no))
  (plugging (front no) (back no)) (filling no) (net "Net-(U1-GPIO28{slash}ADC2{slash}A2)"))
 (via (at 204.378 65.5) (size 0.6) (drill 0.3) (layers "F.Cu" "B.Cu") (capping no) (covering (front no) (back no))
  (plugging (front no) (back no)) (filling no) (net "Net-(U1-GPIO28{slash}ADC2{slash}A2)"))
 (segment (start 204.4 65.5) (end 204.378 65.5) (width 0.2) (layer "B.Cu") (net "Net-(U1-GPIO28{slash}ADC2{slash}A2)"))
 (segment (start 206.3 67.4) (end 204.4 65.5) (width 0.2) (layer "B.Cu") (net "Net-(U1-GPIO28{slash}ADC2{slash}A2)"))
 (segment (start 209.1 85.9) (end 209 85.8) (width 0.2) (layer "F.Cu") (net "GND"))
 (segment (start 219.3 61.4) (end 218.191 61.4) (width 0.2) (layer "F.Cu") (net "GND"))
 (segment (start 218.191 61.4) (end 214.195 57.404) (width 0.2) (layer "F.Cu") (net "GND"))
 (segment (start 219.6 61.7) (end 219.3 61.4) (width 0.2) (layer "F.Cu") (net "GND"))
 (segment (start 211.9 85.9) (end 209.1 85.9) (width 0.2) (layer "F.Cu") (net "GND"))
 (via (at 219.6 61.7) (size 0.6) (drill 0.3) (layers "F.Cu" "B.Cu") (capping no) (covering (front no) (back no))
  (plugging (front no) (back no)) (filling no) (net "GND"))
 (via (at 211.9 85.9) (size 0.6) (drill 0.3) (layers "F.Cu" "B.Cu") (capping no) (covering (front no) (back no))
  (plugging (front no) (back no)) (filling no) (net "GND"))
 (via (at 209 85.8) (size 0.6) (drill 0.3) (layers "F.Cu" "B.Cu") (capping no) (covering (front no) (back no))
  (plugging (front no) (back no)) (filling no) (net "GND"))
 (segment (start 236.728 75.666) (end 229.388 68.326) (width 0.2) (layer "B.Cu") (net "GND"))
 (segment (start 255.778 85.852) (end 236.728 85.852) (width 0.2) (layer "B.Cu") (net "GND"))
 (segment (start 255.778 85.852) (end 257.0125 87.0865) (width 0.2) (layer "B.Cu") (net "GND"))
 (segment (start 217.678 91.478) (end 218.9 92.7) (width 0.2) (layer "B.Cu") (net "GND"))
 (segment (start 238.0125 92.7025) (end 236.728 91.418) (width 0.2) (layer "B.Cu") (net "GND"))
 (segment (start 226.226 68.326) (end 219.6 61.7) (width 0.2) (layer "B.Cu") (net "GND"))
 (segment (start 236.728 91.418) (end 236.728 85.852) (width 0.2) (layer "B.Cu") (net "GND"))
 (segment (start 208.948 85.852) (end 198.628 85.852) (width 0.2) (layer "B.Cu") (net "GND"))
 (segment (start 236.728 85.852) (end 236.728 75.666) (width 0.2) (layer "B.Cu") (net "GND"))
 (segment (start 198.628 91.428) (end 199.9 92.7) (width 0.2) (layer "B.Cu") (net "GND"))
 (segment (start 257.0125 87.0865) (end 257.0125 92.7025) (width 0.2) (layer "B.Cu") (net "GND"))
 (segment (start 211.948 85.852) (end 211.9 85.9) (width 0.2) (layer "B.Cu") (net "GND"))
 (segment (start 217.678 85.852) (end 217.678 91.478) (width 0.2) (layer "B.Cu") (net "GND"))
 (segment (start 217.678 85.852) (end 236.728 85.852) (width 0.2) (layer "B.Cu") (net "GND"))
 (segment (start 209 85.8) (end 208.948 85.852) (width 0.2) (layer "B.Cu") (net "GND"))
 (segment (start 217.678 85.852) (end 211.948 85.852) (width 0.2) (layer "B.Cu") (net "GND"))
 (segment (start 198.628 85.852) (end 198.628 91.428) (width 0.2) (layer "B.Cu") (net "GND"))
 (segment (start 229.388 68.326) (end 226.226 68.326) (width 0.2) (layer "B.Cu") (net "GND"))
 (segment (start 243.1 96.6) (end 224.2 96.6) (width 0.5) (layer "B.Cu") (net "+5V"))
 (segment (start 205.9 96.6) (end 205.9 95) (width 0.5) (layer "B.Cu") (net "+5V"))
 (segment (start 205.9 95) (end 205.1 94.2) (width 0.5) (layer "B.Cu") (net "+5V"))
 (segment (start 243.2125 94.2025) (end 243.2125 96.4875) (width 0.5) (layer "B.Cu") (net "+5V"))
 (segment (start 262.2125 95.2875) (end 260.9 96.6) (width 0.5) (layer "B.Cu") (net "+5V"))
 (segment (start 262.2125 94.2025) (end 262.2125 95.2875) (width 0.5) (layer "B.Cu") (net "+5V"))
 (segment (start 210.7 96.6) (end 205.9 96.6) (width 0.5) (layer "B.Cu") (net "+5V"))
 (segment (start 224.1 94.2) (end 224.1 96.5) (width 0.5) (layer "B.Cu") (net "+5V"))
 (segment (start 260.9 96.6) (end 243.1 96.6) (width 0.5) (layer "B.Cu") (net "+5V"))
 (segment (start 224.2 96.6) (end 210.7 96.6) (width 0.5) (layer "B.Cu") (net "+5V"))
 (segment (start 213.36 54.864) (end 210.7 57.524) (width 0.5) (layer "B.Cu") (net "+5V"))
 (segment (start 243.2125 96.4875) (end 243.1 96.6) (width 0.5) (layer "B.Cu") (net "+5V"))
 (segment (start 210.7 57.524) (end 210.7 96.6) (width 0.5) (layer "B.Cu") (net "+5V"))
 (segment (start 224.1 96.5) (end 224.2 96.6) (width 0.5) (layer "B.Cu") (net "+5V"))
 (segment (start 244.0125 92.7025) (end 245.5125 94.2025) (width 0.2) (layer "B.Cu") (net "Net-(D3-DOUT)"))
 (segment (start 243.2125 92.7025) (end 244.0125 92.7025) (width 0.2) (layer "B.Cu") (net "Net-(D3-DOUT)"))
 (segment (start 245.5125 94.2025) (end 257.0125 94.2025) (width 0.2) (layer "B.Cu") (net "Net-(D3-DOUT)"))
 (segment (start 257.316 78.5) (end 225.131 78.5) (width 0.2) (layer "F.Cu") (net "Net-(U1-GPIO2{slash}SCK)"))
 (segment (start 262.128 83.312) (end 257.316 78.5) (width 0.2) (layer "F.Cu") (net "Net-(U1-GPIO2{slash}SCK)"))
 (segment (start 225.131 78.5) (end 214.195 67.564) (width 0.2) (layer "F.Cu") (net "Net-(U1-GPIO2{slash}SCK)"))
 (segment (start 224.1 92.7) (end 224.9 92.7) (width 0.2) (layer "B.Cu") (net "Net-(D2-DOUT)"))
 (segment (start 226.4025 94.2025) (end 238.0125 94.2025) (width 0.2) (layer "B.Cu") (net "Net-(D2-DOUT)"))
 (segment (start 224.9 92.7) (end 226.4025 94.2025) (width 0.2) (layer "B.Cu") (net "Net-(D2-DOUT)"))
 (segment (start 208.5 92.7) (end 211.8 92.7) (width 0.2) (layer "F.Cu") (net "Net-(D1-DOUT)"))
 (via (at 211.8 92.7) (size 0.6) (drill 0.3) (layers "F.Cu" "B.Cu") (capping no) (covering (front no) (back no))
  (plugging (front no) (back no)) (filling no) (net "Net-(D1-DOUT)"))
 (via (at 208.5 92.7) (size 0.6) (drill 0.3) (layers "F.Cu" "B.Cu") (capping no) (covering (front no) (back no))
  (plugging (front no) (back no)) (filling no) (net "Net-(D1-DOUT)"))
 (segment (start 205.1 92.7) (end 208.5 92.7) (width 0.2) (layer "B.Cu") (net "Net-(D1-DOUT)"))
 (segment (start 213.3 94.2) (end 218.9 94.2) (width 0.2) (layer "B.Cu") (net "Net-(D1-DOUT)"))
 (segment (start 211.8 92.7) (end 213.3 94.2) (width 0.2) (layer "B.Cu") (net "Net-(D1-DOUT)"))
 (segment (start 223.556 80.3) (end 213.36 70.104) (width 0.2) (layer "F.Cu") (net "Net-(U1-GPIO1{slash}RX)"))
 (segment (start 240.066 80.3) (end 223.556 80.3) (width 0.2) (layer "F.Cu") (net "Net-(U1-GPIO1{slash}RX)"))
 (segment (start 243.078 83.312) (end 240.066 80.3) (width 0.2) (layer "F.Cu") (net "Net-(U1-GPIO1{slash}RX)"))
 (segment (start 194 89.1) (end 194 56.9) (width 0.2) (layer "B.Cu") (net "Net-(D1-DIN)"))
 (segment (start 194 56.9) (end 196.036 54.864) (width 0.2) (layer "B.Cu") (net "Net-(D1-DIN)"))
 (segment (start 199.9 94.2) (end 199.1 94.2) (width 0.2) (layer "B.Cu") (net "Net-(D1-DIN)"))
 (segment (start 199.1 94.2) (end 194 89.1) (width 0.2) (layer "B.Cu") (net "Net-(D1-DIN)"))
 (segment (start 196.036 54.864) (end 198.12 54.864) (width 0.2) (layer "B.Cu") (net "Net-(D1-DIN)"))
 (segment (start 204.978 64.262) (end 204.978 83.312) (width 0.2) (layer "F.Cu") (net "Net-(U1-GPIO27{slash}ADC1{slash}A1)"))
 (segment (start 198.12 57.404) (end 204.978 64.262) (width 0.2) (layer "F.Cu") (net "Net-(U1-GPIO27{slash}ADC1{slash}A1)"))
 (segment (start 229.388 60.706) (end 226.133 63.961) (width 0.2) (layer "F.Cu") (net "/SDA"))
 (segment (start 201.4 64.6) (end 200.976 65.024) (width 0.2) (layer "F.Cu") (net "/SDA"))
 (segment (start 200.976 65.024) (end 197.285 65.024) (width 0.2) (layer "F.Cu") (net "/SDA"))
 (segment (start 206.839 63.961) (end 206.3 64.5) (width 0.2) (layer "F.Cu") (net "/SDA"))
 (segment (start 226.133 63.961) (end 206.839 63.961) (width 0.2) (layer "F.Cu") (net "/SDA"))
 (via (at 201.4 64.6) (size 0.6) (drill 0.3) (layers "F.Cu" "B.Cu") (capping no) (covering (front no) (back no))
  (plugging (front no) (back no)) (filling no) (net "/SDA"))
 (via (at 206.3 64.5) (size 0.6) (drill 0.3) (layers "F.Cu" "B.Cu") (capping no) (covering (front no) (back no))
  (plugging (front no) (back no)) (filling no) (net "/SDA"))
 (segment (start 206.3 64.5) (end 201.5 64.5) (width 0.2) (layer "B.Cu") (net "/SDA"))
 (segment (start 201.5 64.5) (end 201.4 64.6) (width 0.2) (layer "B.Cu") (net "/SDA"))
 (segment (start 209.999 66.501) (end 226.133 66.501) (width 0.2) (layer "F.Cu") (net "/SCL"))
 (segment (start 208.3 68.2) (end 209.999 66.501) (width 0.2) (layer "F.Cu") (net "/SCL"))
 (segment (start 203.064 67.564) (end 203.1 67.6) (width 0.2) (layer "F.Cu") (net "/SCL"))
 (segment (start 198.12 67.564) (end 203.064 67.564) (width 0.2) (layer "F.Cu") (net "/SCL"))
 (segment (start 226.133 66.501) (end 229.388 63.246) (width 0.2) (layer "F.Cu") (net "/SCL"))
 (via (at 208.3 68.2) (size 0.6) (drill 0.3) (layers "F.Cu" "B.Cu") (capping no) (covering (front no) (back no))
  (plugging (front no) (back no)) (filling no) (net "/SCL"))
 (via (at 203.1 67.6) (size 0.6) (drill 0.3) (layers "F.Cu" "B.Cu") (capping no) (covering (front no) (back no))
  (plugging (front no) (back no)) (filling no) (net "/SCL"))
 (segment (start 203.1 67.6) (end 203.7 68.2) (width 0.2) (layer "B.Cu") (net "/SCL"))
 (segment (start 203.7 68.2) (end 208.3 68.2) (width 0.2) (layer "B.Cu") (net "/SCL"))
 (segment (start 229.388 65.786) (end 223.546 59.944) (width 0.5) (layer "B.Cu") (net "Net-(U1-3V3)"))
 (segment (start 223.546 59.944) (end 213.36 59.944) (width 0.5) (layer "B.Cu") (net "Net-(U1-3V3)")))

